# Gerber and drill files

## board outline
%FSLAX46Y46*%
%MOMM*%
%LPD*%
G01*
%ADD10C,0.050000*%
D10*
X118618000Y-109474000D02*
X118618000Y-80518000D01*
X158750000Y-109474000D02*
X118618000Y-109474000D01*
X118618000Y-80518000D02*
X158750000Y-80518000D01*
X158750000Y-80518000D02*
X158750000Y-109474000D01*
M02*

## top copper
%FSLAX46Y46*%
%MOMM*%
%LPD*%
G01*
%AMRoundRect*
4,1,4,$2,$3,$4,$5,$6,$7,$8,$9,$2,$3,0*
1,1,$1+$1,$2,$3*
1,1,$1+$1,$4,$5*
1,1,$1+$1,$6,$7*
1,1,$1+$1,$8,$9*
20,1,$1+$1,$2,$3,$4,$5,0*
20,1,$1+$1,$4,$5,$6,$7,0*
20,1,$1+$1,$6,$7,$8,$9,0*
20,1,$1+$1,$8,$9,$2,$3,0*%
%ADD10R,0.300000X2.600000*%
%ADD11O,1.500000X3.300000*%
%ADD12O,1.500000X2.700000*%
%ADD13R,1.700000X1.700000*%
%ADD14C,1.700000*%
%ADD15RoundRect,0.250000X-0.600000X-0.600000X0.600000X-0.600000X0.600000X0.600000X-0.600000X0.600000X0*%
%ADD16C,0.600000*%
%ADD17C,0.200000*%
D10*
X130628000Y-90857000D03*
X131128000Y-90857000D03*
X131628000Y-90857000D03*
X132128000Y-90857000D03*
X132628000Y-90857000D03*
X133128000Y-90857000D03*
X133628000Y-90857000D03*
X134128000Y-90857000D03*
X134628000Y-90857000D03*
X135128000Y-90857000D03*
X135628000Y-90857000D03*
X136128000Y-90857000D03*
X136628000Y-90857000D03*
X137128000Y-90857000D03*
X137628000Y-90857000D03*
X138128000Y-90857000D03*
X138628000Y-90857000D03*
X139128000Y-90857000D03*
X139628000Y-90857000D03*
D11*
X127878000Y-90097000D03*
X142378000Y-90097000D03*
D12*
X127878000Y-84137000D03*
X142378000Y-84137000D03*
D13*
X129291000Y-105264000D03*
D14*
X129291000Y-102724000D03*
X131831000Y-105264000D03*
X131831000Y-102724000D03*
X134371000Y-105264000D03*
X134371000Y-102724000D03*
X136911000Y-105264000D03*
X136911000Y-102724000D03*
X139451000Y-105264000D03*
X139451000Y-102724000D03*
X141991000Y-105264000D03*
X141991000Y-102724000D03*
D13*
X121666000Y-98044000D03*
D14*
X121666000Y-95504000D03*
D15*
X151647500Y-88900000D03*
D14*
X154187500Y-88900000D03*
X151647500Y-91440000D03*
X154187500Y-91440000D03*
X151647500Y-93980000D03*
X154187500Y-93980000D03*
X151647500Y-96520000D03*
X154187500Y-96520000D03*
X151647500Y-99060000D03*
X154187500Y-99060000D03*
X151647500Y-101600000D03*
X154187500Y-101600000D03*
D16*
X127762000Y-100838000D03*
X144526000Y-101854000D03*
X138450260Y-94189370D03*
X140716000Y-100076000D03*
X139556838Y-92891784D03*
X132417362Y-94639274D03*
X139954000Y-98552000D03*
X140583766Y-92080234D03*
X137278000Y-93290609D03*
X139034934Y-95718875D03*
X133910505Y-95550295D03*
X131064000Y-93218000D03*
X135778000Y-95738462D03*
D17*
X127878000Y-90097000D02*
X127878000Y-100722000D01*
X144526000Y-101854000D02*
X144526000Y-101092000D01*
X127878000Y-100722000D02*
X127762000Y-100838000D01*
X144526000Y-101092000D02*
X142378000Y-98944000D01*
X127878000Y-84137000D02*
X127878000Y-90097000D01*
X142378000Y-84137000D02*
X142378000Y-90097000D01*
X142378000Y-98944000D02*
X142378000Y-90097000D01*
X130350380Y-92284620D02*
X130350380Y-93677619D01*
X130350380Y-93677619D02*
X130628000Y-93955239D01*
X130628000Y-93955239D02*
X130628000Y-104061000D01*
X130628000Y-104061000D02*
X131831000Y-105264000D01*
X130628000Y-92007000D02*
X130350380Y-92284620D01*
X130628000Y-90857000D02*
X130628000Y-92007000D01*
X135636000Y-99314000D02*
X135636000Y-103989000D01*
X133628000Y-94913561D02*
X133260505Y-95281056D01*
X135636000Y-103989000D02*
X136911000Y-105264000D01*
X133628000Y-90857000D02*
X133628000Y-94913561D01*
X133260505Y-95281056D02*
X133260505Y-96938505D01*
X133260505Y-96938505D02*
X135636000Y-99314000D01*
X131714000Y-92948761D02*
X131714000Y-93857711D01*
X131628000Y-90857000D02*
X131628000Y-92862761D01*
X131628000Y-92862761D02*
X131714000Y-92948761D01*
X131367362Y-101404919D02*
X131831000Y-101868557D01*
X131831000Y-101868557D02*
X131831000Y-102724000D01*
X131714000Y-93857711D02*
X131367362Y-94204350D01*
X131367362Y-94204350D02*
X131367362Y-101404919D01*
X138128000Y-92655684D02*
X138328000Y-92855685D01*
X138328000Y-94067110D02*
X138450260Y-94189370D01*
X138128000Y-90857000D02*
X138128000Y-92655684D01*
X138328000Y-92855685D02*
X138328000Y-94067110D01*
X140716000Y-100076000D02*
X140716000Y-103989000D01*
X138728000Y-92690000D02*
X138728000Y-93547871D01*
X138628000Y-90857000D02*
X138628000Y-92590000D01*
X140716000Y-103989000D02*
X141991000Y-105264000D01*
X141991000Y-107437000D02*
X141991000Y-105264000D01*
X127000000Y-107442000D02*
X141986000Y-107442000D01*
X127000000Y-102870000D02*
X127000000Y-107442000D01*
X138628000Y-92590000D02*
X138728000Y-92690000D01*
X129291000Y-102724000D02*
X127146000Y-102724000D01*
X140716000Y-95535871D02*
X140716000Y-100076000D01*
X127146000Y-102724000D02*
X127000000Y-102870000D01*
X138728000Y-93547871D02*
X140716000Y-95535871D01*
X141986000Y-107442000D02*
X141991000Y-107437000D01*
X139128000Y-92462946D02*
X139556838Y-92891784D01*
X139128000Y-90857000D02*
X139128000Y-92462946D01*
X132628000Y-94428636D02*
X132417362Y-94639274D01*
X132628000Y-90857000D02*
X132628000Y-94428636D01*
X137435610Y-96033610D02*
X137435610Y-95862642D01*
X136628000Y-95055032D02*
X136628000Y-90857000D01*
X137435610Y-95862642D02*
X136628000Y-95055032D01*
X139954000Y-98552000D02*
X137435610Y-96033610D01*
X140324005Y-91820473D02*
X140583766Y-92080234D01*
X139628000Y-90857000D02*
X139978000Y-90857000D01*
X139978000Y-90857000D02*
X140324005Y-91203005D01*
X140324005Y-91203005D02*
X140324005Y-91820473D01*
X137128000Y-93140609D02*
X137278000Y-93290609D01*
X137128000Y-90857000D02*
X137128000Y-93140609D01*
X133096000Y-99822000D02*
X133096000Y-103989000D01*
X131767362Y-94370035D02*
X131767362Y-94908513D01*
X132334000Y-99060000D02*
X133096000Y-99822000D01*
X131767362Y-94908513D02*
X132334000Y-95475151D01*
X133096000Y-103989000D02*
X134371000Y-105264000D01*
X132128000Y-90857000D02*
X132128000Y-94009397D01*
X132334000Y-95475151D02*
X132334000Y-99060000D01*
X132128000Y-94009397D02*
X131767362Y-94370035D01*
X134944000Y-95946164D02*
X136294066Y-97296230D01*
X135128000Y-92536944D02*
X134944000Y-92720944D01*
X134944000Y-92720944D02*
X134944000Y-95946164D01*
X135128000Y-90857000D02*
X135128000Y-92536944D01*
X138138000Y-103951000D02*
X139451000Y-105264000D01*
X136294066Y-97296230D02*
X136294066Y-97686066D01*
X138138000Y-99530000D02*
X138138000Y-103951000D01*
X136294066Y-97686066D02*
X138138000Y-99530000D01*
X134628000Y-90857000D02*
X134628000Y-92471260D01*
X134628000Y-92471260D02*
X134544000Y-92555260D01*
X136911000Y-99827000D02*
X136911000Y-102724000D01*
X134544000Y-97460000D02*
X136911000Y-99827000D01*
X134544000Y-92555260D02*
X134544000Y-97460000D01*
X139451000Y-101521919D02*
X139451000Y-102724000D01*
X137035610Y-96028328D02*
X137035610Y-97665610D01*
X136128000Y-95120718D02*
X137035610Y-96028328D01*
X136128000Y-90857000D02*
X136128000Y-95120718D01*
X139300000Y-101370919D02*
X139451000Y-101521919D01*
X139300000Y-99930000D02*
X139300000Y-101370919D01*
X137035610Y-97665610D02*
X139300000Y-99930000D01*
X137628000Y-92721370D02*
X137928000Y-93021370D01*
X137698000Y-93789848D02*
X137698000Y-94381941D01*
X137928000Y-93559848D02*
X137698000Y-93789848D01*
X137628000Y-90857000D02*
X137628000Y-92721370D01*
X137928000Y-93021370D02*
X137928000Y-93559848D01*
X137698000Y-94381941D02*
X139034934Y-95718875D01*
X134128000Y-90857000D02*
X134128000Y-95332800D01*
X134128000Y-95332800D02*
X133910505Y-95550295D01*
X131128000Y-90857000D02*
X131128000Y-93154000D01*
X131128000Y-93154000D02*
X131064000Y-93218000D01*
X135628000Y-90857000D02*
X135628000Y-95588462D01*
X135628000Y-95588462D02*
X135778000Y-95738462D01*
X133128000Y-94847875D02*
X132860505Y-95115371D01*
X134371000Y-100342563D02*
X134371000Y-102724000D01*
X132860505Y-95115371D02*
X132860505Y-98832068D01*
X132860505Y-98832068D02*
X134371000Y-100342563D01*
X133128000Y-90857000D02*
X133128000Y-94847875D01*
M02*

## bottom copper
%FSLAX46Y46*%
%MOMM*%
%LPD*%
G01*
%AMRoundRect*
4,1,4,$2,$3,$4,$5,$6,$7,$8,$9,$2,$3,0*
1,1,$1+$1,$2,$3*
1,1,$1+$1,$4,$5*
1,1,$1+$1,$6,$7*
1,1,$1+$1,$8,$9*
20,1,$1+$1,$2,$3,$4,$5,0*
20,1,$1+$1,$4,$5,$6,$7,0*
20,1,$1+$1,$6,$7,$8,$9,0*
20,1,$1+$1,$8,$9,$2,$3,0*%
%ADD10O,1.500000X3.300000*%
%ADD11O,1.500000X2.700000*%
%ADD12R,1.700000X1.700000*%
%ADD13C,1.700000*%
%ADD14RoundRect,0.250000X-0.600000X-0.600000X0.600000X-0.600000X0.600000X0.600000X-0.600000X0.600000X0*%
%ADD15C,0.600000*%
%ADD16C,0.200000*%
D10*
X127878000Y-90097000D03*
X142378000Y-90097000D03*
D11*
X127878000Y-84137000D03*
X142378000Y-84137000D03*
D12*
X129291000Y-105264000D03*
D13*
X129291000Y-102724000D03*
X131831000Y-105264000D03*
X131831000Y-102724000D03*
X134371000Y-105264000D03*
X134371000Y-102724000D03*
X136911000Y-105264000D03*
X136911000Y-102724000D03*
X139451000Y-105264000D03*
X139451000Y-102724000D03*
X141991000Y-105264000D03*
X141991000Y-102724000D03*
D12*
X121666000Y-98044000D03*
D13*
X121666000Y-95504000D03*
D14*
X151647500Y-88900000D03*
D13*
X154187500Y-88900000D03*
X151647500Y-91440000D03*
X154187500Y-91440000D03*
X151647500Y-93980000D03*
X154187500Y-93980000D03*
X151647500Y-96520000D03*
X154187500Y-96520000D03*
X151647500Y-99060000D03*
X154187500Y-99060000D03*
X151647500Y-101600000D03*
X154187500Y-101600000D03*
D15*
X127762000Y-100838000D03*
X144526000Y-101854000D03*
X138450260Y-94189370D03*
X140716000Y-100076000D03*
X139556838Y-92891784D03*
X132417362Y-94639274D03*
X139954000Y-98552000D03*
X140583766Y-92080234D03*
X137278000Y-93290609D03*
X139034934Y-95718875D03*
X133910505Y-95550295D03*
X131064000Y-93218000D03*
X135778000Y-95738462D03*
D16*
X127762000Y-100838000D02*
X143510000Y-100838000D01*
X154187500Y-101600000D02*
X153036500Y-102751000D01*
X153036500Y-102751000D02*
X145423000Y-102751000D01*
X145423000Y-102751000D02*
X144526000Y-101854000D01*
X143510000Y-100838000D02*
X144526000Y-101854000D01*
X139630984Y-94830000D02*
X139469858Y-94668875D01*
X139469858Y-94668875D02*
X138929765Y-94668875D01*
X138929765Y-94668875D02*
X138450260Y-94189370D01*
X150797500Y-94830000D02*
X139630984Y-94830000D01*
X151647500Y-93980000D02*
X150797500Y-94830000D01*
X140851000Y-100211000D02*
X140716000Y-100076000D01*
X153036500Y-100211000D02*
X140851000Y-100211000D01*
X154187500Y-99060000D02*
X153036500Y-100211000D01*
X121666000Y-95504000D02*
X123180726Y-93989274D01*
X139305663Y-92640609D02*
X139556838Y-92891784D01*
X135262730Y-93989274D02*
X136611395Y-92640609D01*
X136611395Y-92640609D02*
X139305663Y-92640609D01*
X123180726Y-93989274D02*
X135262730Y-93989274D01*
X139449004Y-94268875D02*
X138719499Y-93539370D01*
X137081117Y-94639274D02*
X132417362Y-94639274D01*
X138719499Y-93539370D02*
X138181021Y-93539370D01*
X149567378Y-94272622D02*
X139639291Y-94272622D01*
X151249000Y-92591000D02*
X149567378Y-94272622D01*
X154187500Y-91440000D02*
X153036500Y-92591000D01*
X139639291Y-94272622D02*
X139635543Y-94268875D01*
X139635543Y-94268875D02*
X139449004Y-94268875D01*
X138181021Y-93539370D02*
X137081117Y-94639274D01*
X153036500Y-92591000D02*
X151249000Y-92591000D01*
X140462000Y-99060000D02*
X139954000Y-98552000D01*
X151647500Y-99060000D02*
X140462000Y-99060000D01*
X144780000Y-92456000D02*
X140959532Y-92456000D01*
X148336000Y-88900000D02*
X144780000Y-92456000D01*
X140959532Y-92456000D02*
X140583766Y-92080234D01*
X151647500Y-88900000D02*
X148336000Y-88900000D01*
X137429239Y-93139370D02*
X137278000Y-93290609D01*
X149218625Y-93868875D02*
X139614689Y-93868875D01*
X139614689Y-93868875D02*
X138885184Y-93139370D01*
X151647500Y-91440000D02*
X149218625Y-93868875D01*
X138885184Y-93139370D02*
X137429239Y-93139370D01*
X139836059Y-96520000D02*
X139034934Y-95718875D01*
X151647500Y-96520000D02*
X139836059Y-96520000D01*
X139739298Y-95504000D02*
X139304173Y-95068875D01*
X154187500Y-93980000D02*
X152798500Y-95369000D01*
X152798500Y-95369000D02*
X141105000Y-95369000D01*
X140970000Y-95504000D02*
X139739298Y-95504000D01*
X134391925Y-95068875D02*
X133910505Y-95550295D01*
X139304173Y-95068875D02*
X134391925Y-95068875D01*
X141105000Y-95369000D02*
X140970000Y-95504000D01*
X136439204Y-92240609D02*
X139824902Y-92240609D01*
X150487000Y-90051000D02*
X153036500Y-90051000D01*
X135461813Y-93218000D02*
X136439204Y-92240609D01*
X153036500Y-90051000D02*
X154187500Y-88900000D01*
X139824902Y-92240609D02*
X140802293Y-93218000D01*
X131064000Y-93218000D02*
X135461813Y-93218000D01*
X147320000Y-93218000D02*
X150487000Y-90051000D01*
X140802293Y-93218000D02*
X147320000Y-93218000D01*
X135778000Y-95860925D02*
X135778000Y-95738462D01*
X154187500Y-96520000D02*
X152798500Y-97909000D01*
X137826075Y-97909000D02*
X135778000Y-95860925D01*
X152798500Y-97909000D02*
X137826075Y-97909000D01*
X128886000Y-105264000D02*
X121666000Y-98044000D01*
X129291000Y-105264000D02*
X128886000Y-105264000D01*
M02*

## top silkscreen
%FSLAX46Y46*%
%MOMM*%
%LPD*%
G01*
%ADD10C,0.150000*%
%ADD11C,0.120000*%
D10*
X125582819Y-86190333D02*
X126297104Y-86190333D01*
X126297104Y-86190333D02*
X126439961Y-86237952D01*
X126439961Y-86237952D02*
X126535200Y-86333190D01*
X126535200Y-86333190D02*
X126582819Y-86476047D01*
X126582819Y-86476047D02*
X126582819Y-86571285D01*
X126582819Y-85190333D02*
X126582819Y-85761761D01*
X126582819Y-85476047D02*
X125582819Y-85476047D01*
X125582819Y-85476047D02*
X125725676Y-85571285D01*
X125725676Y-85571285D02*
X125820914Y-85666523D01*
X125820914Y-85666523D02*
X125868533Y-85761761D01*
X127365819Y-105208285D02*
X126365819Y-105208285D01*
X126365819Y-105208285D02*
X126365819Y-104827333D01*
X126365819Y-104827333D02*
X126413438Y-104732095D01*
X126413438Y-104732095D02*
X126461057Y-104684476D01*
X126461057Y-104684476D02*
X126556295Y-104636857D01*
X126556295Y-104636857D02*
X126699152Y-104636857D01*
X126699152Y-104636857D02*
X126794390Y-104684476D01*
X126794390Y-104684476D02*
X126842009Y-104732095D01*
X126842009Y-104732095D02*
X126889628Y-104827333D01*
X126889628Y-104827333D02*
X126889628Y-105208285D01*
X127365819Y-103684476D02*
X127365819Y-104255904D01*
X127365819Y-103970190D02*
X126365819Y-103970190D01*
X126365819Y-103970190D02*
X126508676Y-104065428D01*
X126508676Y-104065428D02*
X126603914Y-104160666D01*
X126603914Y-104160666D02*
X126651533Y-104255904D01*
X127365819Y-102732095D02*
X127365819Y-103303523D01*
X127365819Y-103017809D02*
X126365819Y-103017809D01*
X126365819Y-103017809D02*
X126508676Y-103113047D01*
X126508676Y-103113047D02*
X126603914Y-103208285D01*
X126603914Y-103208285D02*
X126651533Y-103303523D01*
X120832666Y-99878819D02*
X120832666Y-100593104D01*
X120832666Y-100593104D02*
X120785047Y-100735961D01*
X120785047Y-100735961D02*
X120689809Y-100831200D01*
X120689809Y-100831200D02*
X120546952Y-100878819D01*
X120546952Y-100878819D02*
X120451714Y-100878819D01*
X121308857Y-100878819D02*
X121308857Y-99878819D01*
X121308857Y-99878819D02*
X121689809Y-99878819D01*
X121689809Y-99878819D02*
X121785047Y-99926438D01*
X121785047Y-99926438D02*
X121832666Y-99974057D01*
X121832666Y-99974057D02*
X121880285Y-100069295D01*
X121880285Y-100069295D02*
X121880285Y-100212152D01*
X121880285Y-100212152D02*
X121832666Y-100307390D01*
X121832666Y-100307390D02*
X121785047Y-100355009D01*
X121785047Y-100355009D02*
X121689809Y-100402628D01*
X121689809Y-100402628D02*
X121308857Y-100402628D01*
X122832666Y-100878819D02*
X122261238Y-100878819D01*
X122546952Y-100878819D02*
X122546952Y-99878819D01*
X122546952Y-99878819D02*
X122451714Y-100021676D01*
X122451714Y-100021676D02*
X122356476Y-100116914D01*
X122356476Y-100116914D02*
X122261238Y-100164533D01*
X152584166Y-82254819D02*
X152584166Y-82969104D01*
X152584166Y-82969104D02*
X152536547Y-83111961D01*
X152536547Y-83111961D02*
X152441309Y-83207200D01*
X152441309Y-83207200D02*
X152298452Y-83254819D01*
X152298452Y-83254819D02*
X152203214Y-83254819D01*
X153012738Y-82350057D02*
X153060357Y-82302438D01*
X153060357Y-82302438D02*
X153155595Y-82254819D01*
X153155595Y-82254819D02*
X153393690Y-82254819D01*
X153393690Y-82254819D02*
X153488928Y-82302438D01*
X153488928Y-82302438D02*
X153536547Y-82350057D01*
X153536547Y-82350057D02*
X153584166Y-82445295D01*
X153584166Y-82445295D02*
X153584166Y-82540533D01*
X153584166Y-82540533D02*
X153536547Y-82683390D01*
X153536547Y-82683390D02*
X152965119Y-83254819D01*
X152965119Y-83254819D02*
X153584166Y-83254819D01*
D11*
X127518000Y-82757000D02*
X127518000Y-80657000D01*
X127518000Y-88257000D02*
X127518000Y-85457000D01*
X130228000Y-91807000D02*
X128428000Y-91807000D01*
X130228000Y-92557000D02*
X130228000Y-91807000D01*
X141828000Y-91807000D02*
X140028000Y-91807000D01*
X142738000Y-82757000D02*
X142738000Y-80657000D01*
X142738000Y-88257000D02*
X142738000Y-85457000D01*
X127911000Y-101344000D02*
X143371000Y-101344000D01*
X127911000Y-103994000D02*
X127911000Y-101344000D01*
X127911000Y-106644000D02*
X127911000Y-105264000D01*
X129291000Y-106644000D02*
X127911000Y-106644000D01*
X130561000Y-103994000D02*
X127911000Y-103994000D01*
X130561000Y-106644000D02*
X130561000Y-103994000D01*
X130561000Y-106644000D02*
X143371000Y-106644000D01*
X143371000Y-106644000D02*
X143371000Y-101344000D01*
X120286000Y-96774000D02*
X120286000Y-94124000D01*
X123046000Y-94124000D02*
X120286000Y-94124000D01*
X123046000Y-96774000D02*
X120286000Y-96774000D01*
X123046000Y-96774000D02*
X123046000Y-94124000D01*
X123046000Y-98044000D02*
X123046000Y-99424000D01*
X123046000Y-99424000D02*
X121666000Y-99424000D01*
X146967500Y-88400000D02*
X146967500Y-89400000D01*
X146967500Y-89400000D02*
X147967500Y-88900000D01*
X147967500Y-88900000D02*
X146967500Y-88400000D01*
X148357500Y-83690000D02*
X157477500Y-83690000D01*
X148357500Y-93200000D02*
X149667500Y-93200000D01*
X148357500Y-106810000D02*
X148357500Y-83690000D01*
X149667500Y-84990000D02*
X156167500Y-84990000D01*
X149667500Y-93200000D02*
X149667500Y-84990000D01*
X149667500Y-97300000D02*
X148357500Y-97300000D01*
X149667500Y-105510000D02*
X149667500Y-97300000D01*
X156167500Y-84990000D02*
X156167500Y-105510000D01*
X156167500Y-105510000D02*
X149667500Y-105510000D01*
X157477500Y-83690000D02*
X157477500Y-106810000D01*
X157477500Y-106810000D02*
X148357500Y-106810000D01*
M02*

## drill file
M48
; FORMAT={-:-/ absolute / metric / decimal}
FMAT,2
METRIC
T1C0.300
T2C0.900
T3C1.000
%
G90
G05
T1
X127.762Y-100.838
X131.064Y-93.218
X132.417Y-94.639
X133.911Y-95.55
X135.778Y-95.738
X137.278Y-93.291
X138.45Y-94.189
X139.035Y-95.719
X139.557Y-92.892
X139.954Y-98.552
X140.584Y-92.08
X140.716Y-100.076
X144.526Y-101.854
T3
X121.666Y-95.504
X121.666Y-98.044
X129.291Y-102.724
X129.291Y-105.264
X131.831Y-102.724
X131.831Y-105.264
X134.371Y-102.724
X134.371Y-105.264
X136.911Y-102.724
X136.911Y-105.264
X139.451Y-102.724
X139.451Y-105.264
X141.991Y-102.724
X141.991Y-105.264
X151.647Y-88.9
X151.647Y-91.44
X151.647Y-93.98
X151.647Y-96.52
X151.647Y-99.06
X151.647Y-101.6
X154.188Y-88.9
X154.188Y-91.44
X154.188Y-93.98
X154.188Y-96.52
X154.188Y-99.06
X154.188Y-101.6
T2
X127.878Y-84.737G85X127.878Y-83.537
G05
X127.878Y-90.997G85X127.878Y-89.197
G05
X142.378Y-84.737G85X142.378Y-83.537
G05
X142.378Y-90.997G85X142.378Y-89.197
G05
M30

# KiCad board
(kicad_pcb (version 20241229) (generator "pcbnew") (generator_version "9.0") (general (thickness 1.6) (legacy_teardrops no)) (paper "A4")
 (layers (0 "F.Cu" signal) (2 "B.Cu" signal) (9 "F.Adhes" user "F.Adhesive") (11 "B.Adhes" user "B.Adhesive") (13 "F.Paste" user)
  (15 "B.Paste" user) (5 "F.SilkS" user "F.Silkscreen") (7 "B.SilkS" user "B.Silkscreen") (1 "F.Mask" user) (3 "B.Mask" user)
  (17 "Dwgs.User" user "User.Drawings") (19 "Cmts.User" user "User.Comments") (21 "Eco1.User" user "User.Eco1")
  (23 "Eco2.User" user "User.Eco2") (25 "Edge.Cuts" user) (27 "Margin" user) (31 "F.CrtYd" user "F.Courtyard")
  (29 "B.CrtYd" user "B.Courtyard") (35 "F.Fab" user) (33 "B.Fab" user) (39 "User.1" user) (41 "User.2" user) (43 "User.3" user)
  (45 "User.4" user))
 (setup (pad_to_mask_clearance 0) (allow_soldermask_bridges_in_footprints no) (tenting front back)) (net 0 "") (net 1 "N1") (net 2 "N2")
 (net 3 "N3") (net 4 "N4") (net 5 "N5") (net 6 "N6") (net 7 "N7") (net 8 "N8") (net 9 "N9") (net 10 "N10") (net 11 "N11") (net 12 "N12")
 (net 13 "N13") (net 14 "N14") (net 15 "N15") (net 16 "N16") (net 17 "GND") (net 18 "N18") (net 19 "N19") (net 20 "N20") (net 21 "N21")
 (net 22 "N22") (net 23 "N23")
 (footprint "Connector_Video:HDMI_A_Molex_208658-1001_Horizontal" (layer "F.Cu") (at 135.128 87.572 90)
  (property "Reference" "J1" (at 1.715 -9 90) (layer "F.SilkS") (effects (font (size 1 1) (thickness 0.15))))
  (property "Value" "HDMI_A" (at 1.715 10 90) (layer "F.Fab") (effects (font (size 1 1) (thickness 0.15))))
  (fp_line (start 4.815 -7.61) (end 6.915 -7.61) (stroke (width 0.12) (type solid)) (layer "F.SilkS"))
  (fp_line (start -0.685 -7.61) (end 2.115 -7.61) (stroke (width 0.12) (type solid)) (layer "F.SilkS"))
  (fp_line (start -4.235 -4.9) (end -4.235 -6.7) (stroke (width 0.12) (type solid)) (layer "F.SilkS"))
  (fp_line (start -4.985 -4.9) (end -4.235 -4.9) (stroke (width 0.12) (type solid)) (layer "F.SilkS"))
  (fp_line (start -4.235 6.7) (end -4.235 4.9) (stroke (width 0.12) (type solid)) (layer "F.SilkS"))
  (fp_line (start 4.815 7.61) (end 6.915 7.61) (stroke (width 0.12) (type solid)) (layer "F.SilkS"))
  (fp_line (start -0.685 7.61) (end 2.115 7.61) (stroke (width 0.12) (type solid)) (layer "F.SilkS"))
  (pad "1" smd rect (at -3.285 -4.5 90) (size 2.6 0.3) (layers "F.Cu" "F.Mask" "F.Paste") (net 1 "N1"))
  (pad "2" smd rect (at -3.285 -4 90) (size 2.6 0.3) (layers "F.Cu" "F.Mask" "F.Paste") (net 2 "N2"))
  (pad "3" smd rect (at -3.285 -3.5 90) (size 2.6 0.3) (layers "F.Cu" "F.Mask" "F.Paste") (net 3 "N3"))
  (pad "4" smd rect (at -3.285 -3 90) (size 2.6 0.3) (layers "F.Cu" "F.Mask" "F.Paste") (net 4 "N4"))
  (pad "5" smd rect (at -3.285 -2.5 90) (size 2.6 0.3) (layers "F.Cu" "F.Mask" "F.Paste") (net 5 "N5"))
  (pad "6" smd rect (at -3.285 -2 90) (size 2.6 0.3) (layers "F.Cu" "F.Mask" "F.Paste") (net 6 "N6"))
  (pad "7" smd rect (at -3.285 -1.5 90) (size 2.6 0.3) (layers "F.Cu" "F.Mask" "F.Paste") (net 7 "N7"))
  (pad "8" smd rect (at -3.285 -1 90) (size 2.6 0.3) (layers "F.Cu" "F.Mask" "F.Paste") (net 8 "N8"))
  (pad "9" smd rect (at -3.285 -0.5 90) (size 2.6 0.3) (layers "F.Cu" "F.Mask" "F.Paste") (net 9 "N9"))
  (pad "10" smd rect (at -3.285 0 90) (size 2.6 0.3) (layers "F.Cu" "F.Mask" "F.Paste") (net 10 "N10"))
  (pad "11" smd rect (at -3.285 0.5 90) (size 2.6 0.3) (layers "F.Cu" "F.Mask" "F.Paste") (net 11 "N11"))
  (pad "12" smd rect (at -3.285 1 90) (size 2.6 0.3) (layers "F.Cu" "F.Mask" "F.Paste") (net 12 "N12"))
  (pad "13" smd rect (at -3.285 1.5 90) (size 2.6 0.3) (layers "F.Cu" "F.Mask" "F.Paste") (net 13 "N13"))
  (pad "14" smd rect (at -3.285 2 90) (size 2.6 0.3) (layers "F.Cu" "F.Mask" "F.Paste") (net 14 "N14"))
  (pad "15" smd rect (at -3.285 2.5 90) (size 2.6 0.3) (layers "F.Cu" "F.Mask" "F.Paste") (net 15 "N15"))
  (pad "16" smd rect (at -3.285 3 90) (size 2.6 0.3) (layers "F.Cu" "F.Mask" "F.Paste") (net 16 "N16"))
  (pad "17" smd rect (at -3.285 3.5 90) (size 2.6 0.3) (layers "F.Cu" "F.Mask" "F.Paste") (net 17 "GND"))
  (pad "18" smd rect (at -3.285 4 90) (size 2.6 0.3) (layers "F.Cu" "F.Mask" "F.Paste") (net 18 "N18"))
  (pad "19" smd rect (at -3.285 4.5 90) (size 2.6 0.3) (layers "F.Cu" "F.Mask" "F.Paste") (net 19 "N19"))
  (pad "SH" thru_hole oval (at -2.525 -7.25 90) (size 3.3 1.5) (drill oval 2.7 0.9) (layers "*.Cu" "*.Mask") (remove_unused_layers no)
   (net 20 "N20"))
  (pad "SH" thru_hole oval (at -2.525 7.25 90) (size 3.3 1.5) (drill oval 2.7 0.9) (layers "*.Cu" "*.Mask") (remove_unused_layers no)
   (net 20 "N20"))
  (pad "SH" thru_hole oval (at 3.435 -7.25 90) (size 2.7 1.5) (drill oval 2.1 0.9) (layers "*.Cu" "*.Mask") (remove_unused_layers no)
   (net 20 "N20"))
  (pad "SH" thru_hole oval (at 3.435 7.25 90) (size 2.7 1.5) (drill oval 2.1 0.9) (layers "*.Cu" "*.Mask") (remove_unused_layers no)
   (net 20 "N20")))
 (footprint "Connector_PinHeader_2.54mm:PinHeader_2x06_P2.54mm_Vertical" (layer "F.Cu") (at 129.291 105.264 90)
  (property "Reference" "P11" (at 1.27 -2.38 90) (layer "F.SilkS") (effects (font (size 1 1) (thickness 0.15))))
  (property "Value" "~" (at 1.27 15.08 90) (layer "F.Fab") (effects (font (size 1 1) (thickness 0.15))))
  (fp_line (start 3.92 -1.38) (end 3.92 14.08) (stroke (width 0.12) (type solid)) (layer "F.SilkS"))
  (fp_line (start 1.27 -1.38) (end 3.92 -1.38) (stroke (width 0.12) (type solid)) (layer "F.SilkS"))
  (fp_line (start -1.38 -1.38) (end 0 -1.38) (stroke (width 0.12) (type solid)) (layer "F.SilkS"))
  (fp_line (start -1.38 0) (end -1.38 -1.38) (stroke (width 0.12) (type solid)) (layer "F.SilkS"))
  (fp_line (start 1.27 1.27) (end 1.27 -1.38) (stroke (width 0.12) (type solid)) (layer "F.SilkS"))
  (fp_line (start -1.38 1.27) (end 1.27 1.27) (stroke (width 0.12) (type solid)) (layer "F.SilkS"))
  (fp_line (start -1.38 1.27) (end -1.38 14.08) (stroke (width 0.12) (type solid)) (layer "F.SilkS"))
  (fp_line (start -1.38 14.08) (end 3.92 14.08) (stroke (width 0.12) (type solid)) (layer "F.SilkS"))
  (pad "1" thru_hole rect (at 0 0 90) (size 1.7 1.7) (drill 1) (layers "*.Cu" "*.Mask") (remove_unused_layers no) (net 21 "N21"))
  (pad "2" thru_hole circle (at 2.54 0 90) (size 1.7 1.7) (drill 1) (layers "*.Cu" "*.Mask") (remove_unused_layers no) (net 17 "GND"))
  (pad "3" thru_hole circle (at 0 2.54 90) (size 1.7 1.7) (drill 1) (layers "*.Cu" "*.Mask") (remove_unused_layers no) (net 1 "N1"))
  (pad "4" thru_hole circle (at 2.54 2.54 90) (size 1.7 1.7) (drill 1) (layers "*.Cu" "*.Mask") (remove_unused_layers no) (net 3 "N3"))
  (pad "5" thru_hole circle (at 0 5.08 90) (size 1.7 1.7) (drill 1) (layers "*.Cu" "*.Mask") (remove_unused_layers no) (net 4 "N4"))
  (pad "6" thru_hole circle (at 2.54 5.08 90) (size 1.7 1.7) (drill 1) (layers "*.Cu" "*.Mask") (remove_unused_layers no) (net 6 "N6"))
  (pad "7" thru_hole circle (at 0 7.62 90) (size 1.7 1.7) (drill 1) (layers "*.Cu" "*.Mask") (remove_unused_layers no) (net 7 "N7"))
  (pad "8" thru_hole circle (at 2.54 7.62 90) (size 1.7 1.7) (drill 1) (layers "*.Cu" "*.Mask") (remove_unused_layers no) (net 9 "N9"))
  (pad "9" thru_hole circle (at 0 10.16 90) (size 1.7 1.7) (drill 1) (layers "*.Cu" "*.Mask") (remove_unused_layers no) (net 10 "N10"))
  (pad "10" thru_hole circle (at 2.54 10.16 90) (size 1.7 1.7) (drill 1) (layers "*.Cu" "*.Mask") (remove_unused_layers no) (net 12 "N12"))
  (pad "11" thru_hole circle (at 0 12.7 90) (size 1.7 1.7) (drill 1) (layers "*.Cu" "*.Mask") (remove_unused_layers no) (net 17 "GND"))
  (pad "12" thru_hole circle (at 2.54 12.7 90) (size 1.7 1.7) (drill 1) (layers "*.Cu" "*.Mask") (remove_unused_layers no) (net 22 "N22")))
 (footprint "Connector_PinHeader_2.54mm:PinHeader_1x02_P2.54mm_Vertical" (layer "F.Cu") (at 121.666 98.044 180)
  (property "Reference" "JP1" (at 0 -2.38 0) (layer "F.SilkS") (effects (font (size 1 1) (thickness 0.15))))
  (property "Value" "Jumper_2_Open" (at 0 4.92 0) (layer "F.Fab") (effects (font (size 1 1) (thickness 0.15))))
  (fp_line (start 1.38 1.27) (end 1.38 3.92) (stroke (width 0.12) (type solid)) (layer "F.SilkS"))
  (fp_line (start -1.38 3.92) (end 1.38 3.92) (stroke (width 0.12) (type solid)) (layer "F.SilkS"))
  (fp_line (start -1.38 1.27) (end 1.38 1.27) (stroke (width 0.12) (type solid)) (layer "F.SilkS"))
  (fp_line (start -1.38 1.27) (end -1.38 3.92) (stroke (width 0.12) (type solid)) (layer "F.SilkS"))
  (fp_line (start -1.38 0) (end -1.38 -1.38) (stroke (width 0.12) (type solid)) (layer "F.SilkS"))
  (fp_line (start -1.38 -1.38) (end 0 -1.38) (stroke (width 0.12) (type solid)) (layer "F.SilkS"))
  (pad "1" thru_hole rect (at 0 0 180) (size 1.7 1.7) (drill 1) (layers "*.Cu" "*.Mask") (remove_unused_layers no) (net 21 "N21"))
  (pad "2" thru_hole circle (at 0 2.54 180) (size 1.7 1.7) (drill 1) (layers "*.Cu" "*.Mask") (remove_unused_layers no) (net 18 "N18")))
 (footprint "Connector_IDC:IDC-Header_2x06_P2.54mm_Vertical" (layer "F.Cu") (at 151.6475 88.9)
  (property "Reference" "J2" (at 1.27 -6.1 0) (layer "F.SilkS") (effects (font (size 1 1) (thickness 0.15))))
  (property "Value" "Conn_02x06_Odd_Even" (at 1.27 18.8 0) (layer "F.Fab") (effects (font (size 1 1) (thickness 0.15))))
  (fp_line (start -4.68 -0.5) (end -4.68 0.5) (stroke (width 0.12) (type solid)) (layer "F.SilkS"))
  (fp_line (start -4.68 0.5) (end -3.68 0) (stroke (width 0.12) (type solid)) (layer "F.SilkS"))
  (fp_line (start -3.68 0) (end -4.68 -0.5) (stroke (width 0.12) (type solid)) (layer "F.SilkS"))
  (fp_line (start -3.29 -5.21) (end 5.83 -5.21) (stroke (width 0.12) (type solid)) (layer "F.SilkS"))
  (fp_line (start -3.29 4.3) (end -1.98 4.3) (stroke (width 0.12) (type solid)) (layer "F.SilkS"))
  (fp_line (start -3.29 17.91) (end -3.29 -5.21) (stroke (width 0.12) (type solid)) (layer "F.SilkS"))
  (fp_line (start -1.98 -3.91) (end 4.52 -3.91) (stroke (width 0.12) (type solid)) (layer "F.SilkS"))
  (fp_line (start -1.98 4.3) (end -1.98 -3.91) (stroke (width 0.12) (type solid)) (layer "F.SilkS"))
  (fp_line (start -1.98 8.4) (end -3.29 8.4) (stroke (width 0.12) (type solid)) (layer "F.SilkS"))
  (fp_line (start -1.98 16.61) (end -1.98 8.4) (stroke (width 0.12) (type solid)) (layer "F.SilkS"))
  (fp_line (start 4.52 -3.91) (end 4.52 16.61) (stroke (width 0.12) (type solid)) (layer "F.SilkS"))
  (fp_line (start 4.52 16.61) (end -1.98 16.61) (stroke (width 0.12) (type solid)) (layer "F.SilkS"))
  (fp_line (start 5.83 -5.21) (end 5.83 17.91) (stroke (width 0.12) (type solid)) (layer "F.SilkS"))
  (fp_line (start 5.83 17.91) (end -3.29 17.91) (stroke (width 0.12) (type solid)) (layer "F.SilkS"))
  (pad "1" thru_hole roundrect (at 0 0) (size 1.7 1.7) (drill 1) (layers "*.Cu" "*.Mask") (remove_unused_layers no)
   (roundrect_rratio 0.147059) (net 19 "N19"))
  (pad "2" thru_hole circle (at 2.54 0) (size 1.7 1.7) (drill 1) (layers "*.Cu" "*.Mask") (remove_unused_layers no) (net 2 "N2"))
  (pad "3" thru_hole circle (at 0 2.54) (size 1.7 1.7) (drill 1) (layers "*.Cu" "*.Mask") (remove_unused_layers no) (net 14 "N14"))
  (pad "4" thru_hole circle (at 2.54 2.54) (size 1.7 1.7) (drill 1) (layers "*.Cu" "*.Mask") (remove_unused_layers no) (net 5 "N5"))
  (pad "5" thru_hole circle (at 0 5.08) (size 1.7 1.7) (drill 1) (layers "*.Cu" "*.Mask") (remove_unused_layers no) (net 16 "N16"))
  (pad "6" thru_hole circle (at 2.54 5.08) (size 1.7 1.7) (drill 1) (layers "*.Cu" "*.Mask") (remove_unused_layers no) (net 8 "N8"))
  (pad "7" thru_hole circle (at 0 7.62) (size 1.7 1.7) (drill 1) (layers "*.Cu" "*.Mask") (remove_unused_layers no) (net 15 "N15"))
  (pad "8" thru_hole circle (at 2.54 7.62) (size 1.7 1.7) (drill 1) (layers "*.Cu" "*.Mask") (remove_unused_layers no) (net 11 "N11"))
  (pad "9" thru_hole circle (at 0 10.16) (size 1.7 1.7) (drill 1) (layers "*.Cu" "*.Mask") (remove_unused_layers no) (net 13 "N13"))
  (pad "10" thru_hole circle (at 2.54 10.16) (size 1.7 1.7) (drill 1) (layers "*.Cu" "*.Mask") (remove_unused_layers no) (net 17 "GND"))
  (pad "11" thru_hole circle (at 0 12.7) (size 1.7 1.7) (drill 1) (layers "*.Cu" "*.Mask") (remove_unused_layers no) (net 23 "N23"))
  (pad "12" thru_hole circle (at 2.54 12.7) (size 1.7 1.7) (drill 1) (layers "*.Cu" "*.Mask") (remove_unused_layers no) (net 20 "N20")))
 (gr_line (start 118.618 109.474) (end 118.618 80.518) (stroke (width 0.05) (type default)) (layer "Edge.Cuts"))
 (gr_line (start 158.75 109.474) (end 118.618 109.474) (stroke (width 0.05) (type default)) (layer "Edge.Cuts"))
 (gr_line (start 118.618 80.518) (end 158.75 80.518) (stroke (width 0.05) (type default)) (layer "Edge.Cuts"))
 (gr_line (start 158.75 80.518) (end 158.75 109.474) (stroke (width 0.05) (type default)) (layer "Edge.Cuts"))
 (segment (start 127.878 90.097) (end 127.878 100.722) (width 0.2) (layer "F.Cu") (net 20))
 (segment (start 144.526 101.854) (end 144.526 101.092) (width 0.2) (layer "F.Cu") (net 20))
 (segment (start 127.878 100.722) (end 127.762 100.838) (width 0.2) (layer "F.Cu") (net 20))
 (segment (start 144.526 101.092) (end 142.378 98.944) (width 0.2) (layer "F.Cu") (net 20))
 (segment (start 127.878 84.137) (end 127.878 90.097) (width 0.2) (layer "F.Cu") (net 20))
 (segment (start 142.378 84.137) (end 142.378 90.097) (width 0.2) (layer "F.Cu") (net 20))
 (segment (start 142.378 98.944) (end 142.378 90.097) (width 0.2) (layer "F.Cu") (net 20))
 (via (at 127.762 100.838) (size 0.6) (drill 0.3) (layers "F.Cu" "B.Cu") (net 20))
 (via (at 144.526 101.854) (size 0.6) (drill 0.3) (layers "F.Cu" "B.Cu") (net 20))
 (segment (start 127.762 100.838) (end 143.51 100.838) (width 0.2) (layer "B.Cu") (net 20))
 (segment (start 154.1875 101.6) (end 153.0365 102.751) (width 0.2) (layer "B.Cu") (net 20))
 (segment (start 153.0365 102.751) (end 145.423 102.751) (width 0.2) (layer "B.Cu") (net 20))
 (segment (start 145.423 102.751) (end 144.526 101.854) (width 0.2) (layer "B.Cu") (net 20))
 (segment (start 143.51 100.838) (end 144.526 101.854) (width 0.2) (layer "B.Cu") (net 20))
 (segment (start 130.35038 92.28462) (end 130.35038 93.677619) (width 0.2) (layer "F.Cu") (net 1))
 (segment (start 130.35038 93.677619) (end 130.628 93.955239) (width 0.2) (layer "F.Cu") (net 1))
 (segment (start 130.628 93.955239) (end 130.628 104.061) (width 0.2) (layer "F.Cu") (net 1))
 (segment (start 130.628 104.061) (end 131.831 105.264) (width 0.2) (layer "F.Cu") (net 1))
 (segment (start 130.628 92.007) (end 130.35038 92.28462) (width 0.2) (layer "F.Cu") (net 1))
 (segment (start 130.628 90.857) (end 130.628 92.007) (width 0.2) (layer "F.Cu") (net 1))
 (segment (start 135.636 99.314) (end 135.636 103.989) (width 0.2) (layer "F.Cu") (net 7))
 (segment (start 133.628 94.913561) (end 133.260505 95.281056) (width 0.2) (layer "F.Cu") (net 7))
 (segment (start 135.636 103.989) (end 136.911 105.264) (width 0.2) (layer "F.Cu") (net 7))
 (segment (start 133.628 90.857) (end 133.628 94.913561) (width 0.2) (layer "F.Cu") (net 7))
 (segment (start 133.260505 95.281056) (end 133.260505 96.938505) (width 0.2) (layer "F.Cu") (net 7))
 (segment (start 133.260505 96.938505) (end 135.636 99.314) (width 0.2) (layer "F.Cu") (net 7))
 (segment (start 131.714 92.948761) (end 131.714 93.857711) (width 0.2) (layer "F.Cu") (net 3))
 (segment (start 131.628 90.857) (end 131.628 92.862761) (width 0.2) (layer "F.Cu") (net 3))
 (segment (start 131.628 92.862761) (end 131.714 92.948761) (width 0.2) (layer "F.Cu") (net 3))
 (segment (start 131.367362 101.404919) (end 131.831 101.868557) (width 0.2) (layer "F.Cu") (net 3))
 (segment (start 131.831 101.868557) (end 131.831 102.724) (width 0.2) (layer "F.Cu") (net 3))
 (segment (start 131.714 93.857711) (end 131.367362 94.20435) (width 0.2) (layer "F.Cu") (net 3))
 (segment (start 131.367362 94.20435) (end 131.367362 101.404919) (width 0.2) (layer "F.Cu") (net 3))
 (segment (start 138.128 92.655684) (end 138.328 92.855685) (width 0.2) (layer "F.Cu") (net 16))
 (segment (start 138.328 94.06711) (end 138.45026 94.18937) (width 0.2) (layer "F.Cu") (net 16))
 (segment (start 138.128 90.857) (end 138.128 92.655684) (width 0.2) (layer "F.Cu") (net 16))
 (segment (start 138.328 92.855685) (end 138.328 94.06711) (width 0.2) (layer "F.Cu") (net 16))
 (via (at 138.45026 94.18937) (size 0.6) (drill 0.3) (layers "F.Cu" "B.Cu") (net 16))
 (segment (start 139.630984 94.83) (end 139.469858 94.668875) (width 0.2) (layer "B.Cu") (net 16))
 (segment (start 139.469858 94.668875) (end 138.929765 94.668875) (width 0.2) (layer "B.Cu") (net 16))
 (segment (start 138.929765 94.668875) (end 138.45026 94.18937) (width 0.2) (layer "B.Cu") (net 16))
 (segment (start 150.7975 94.83) (end 139.630984 94.83) (width 0.2) (layer "B.Cu") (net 16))
 (segment (start 151.6475 93.98) (end 150.7975 94.83) (width 0.2) (layer "B.Cu") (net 16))
 (segment (start 140.716 100.076) (end 140.716 103.989) (width 0.2) (layer "F.Cu") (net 17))
 (segment (start 138.728 92.69) (end 138.728 93.547871) (width 0.2) (layer "F.Cu") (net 17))
 (segment (start 138.628 90.857) (end 138.628 92.59) (width 0.2) (layer "F.Cu") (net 17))
 (segment (start 140.716 103.989) (end 141.991 105.264) (width 0.2) (layer "F.Cu") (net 17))
 (segment (start 141.991 107.437) (end 141.991 105.264) (width 0.2) (layer "F.Cu") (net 17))
 (segment (start 127 107.442) (end 141.986 107.442) (width 0.2) (layer "F.Cu") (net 17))
 (segment (start 127 102.87) (end 127 107.442) (width 0.2) (layer "F.Cu") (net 17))
 (segment (start 138.628 92.59) (end 138.728 92.69) (width 0.2) (layer "F.Cu") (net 17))
 (segment (start 129.291 102.724) (end 127.146 102.724) (width 0.2) (layer "F.Cu") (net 17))
 (segment (start 140.716 95.535871) (end 140.716 100.076) (width 0.2) (layer "F.Cu") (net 17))
 (segment (start 127.146 102.724) (end 127 102.87) (width 0.2) (layer "F.Cu") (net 17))
 (segment (start 138.728 93.547871) (end 140.716 95.535871) (width 0.2) (layer "F.Cu") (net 17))
 (segment (start 141.986 107.442) (end 141.991 107.437) (width 0.2) (layer "F.Cu") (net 17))
 (via (at 140.716 100.076) (size 0.6) (drill 0.3) (layers "F.Cu" "B.Cu") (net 17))
 (segment (start 140.851 100.211) (end 140.716 100.076) (width 0.2) (layer "B.Cu") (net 17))
 (segment (start 153.0365 100.211) (end 140.851 100.211) (width 0.2) (layer "B.Cu") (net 17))
 (segment (start 154.1875 99.06) (end 153.0365 100.211) (width 0.2) (layer "B.Cu") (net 17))
 (segment (start 139.128 92.462946) (end 139.556838 92.891784) (width 0.2) (layer "F.Cu") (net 18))
 (segment (start 139.128 90.857) (end 139.128 92.462946) (width 0.2) (layer "F.Cu") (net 18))
 (via (at 139.556838 92.891784) (size 0.6) (drill 0.3) (layers "F.Cu" "B.Cu") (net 18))
 (segment (start 121.666 95.504) (end 123.180726 93.989274) (width 0.2) (layer "B.Cu") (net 18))
 (segment (start 139.305663 92.640609) (end 139.556838 92.891784) (width 0.2) (layer "B.Cu") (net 18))
 (segment (start 135.26273 93.989274) (end 136.611395 92.640609) (width 0.2) (layer "B.Cu") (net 18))
 (segment (start 136.611395 92.640609) (end 139.305663 92.640609) (width 0.2) (layer "B.Cu") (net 18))
 (segment (start 123.180726 93.989274) (end 135.26273 93.989274) (width 0.2) (layer "B.Cu") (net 18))
 (segment (start 132.628 94.428636) (end 132.417362 94.639274) (width 0.2) (layer "F.Cu") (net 5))
 (segment (start 132.628 90.857) (end 132.628 94.428636) (width 0.2) (layer "F.Cu") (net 5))
 (via (at 132.417362 94.639274) (size 0.6) (drill 0.3) (layers "F.Cu" "B.Cu") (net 5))
 (segment (start 139.449004 94.268875) (end 138.719499 93.53937) (width 0.2) (layer "B.Cu") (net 5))
 (segment (start 137.081117 94.639274) (end 132.417362 94.639274) (width 0.2) (layer "B.Cu") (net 5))
 (segment (start 138.719499 93.53937) (end 138.181021 93.53937) (width 0.2) (layer "B.Cu") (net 5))
 (segment (start 149.567378 94.272622) (end 139.639291 94.272622) (width 0.2) (layer "B.Cu") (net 5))
 (segment (start 151.249 92.591) (end 149.567378 94.272622) (width 0.2) (layer "B.Cu") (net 5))
 (segment (start 154.1875 91.44) (end 153.0365 92.591) (width 0.2) (layer "B.Cu") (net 5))
 (segment (start 139.639291 94.272622) (end 139.635543 94.268875) (width 0.2) (layer "B.Cu") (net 5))
 (segment (start 139.635543 94.268875) (end 139.449004 94.268875) (width 0.2) (layer "B.Cu") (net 5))
 (segment (start 138.181021 93.53937) (end 137.081117 94.639274) (width 0.2) (layer "B.Cu") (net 5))
 (segment (start 153.0365 92.591) (end 151.249 92.591) (width 0.2) (layer "B.Cu") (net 5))
 (segment (start 137.43561 96.03361) (end 137.43561 95.862642) (width 0.2) (layer "F.Cu") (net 13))
 (segment (start 136.628 95.055032) (end 136.628 90.857) (width 0.2) (layer "F.Cu") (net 13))
 (segment (start 137.43561 95.862642) (end 136.628 95.055032) (width 0.2) (layer "F.Cu") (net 13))
 (segment (start 139.954 98.552) (end 137.43561 96.03361) (width 0.2) (layer "F.Cu") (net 13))
 (via (at 139.954 98.552) (size 0.6) (drill 0.3) (layers "F.Cu" "B.Cu") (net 13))
 (segment (start 140.462 99.06) (end 139.954 98.552) (width 0.2) (layer "B.Cu") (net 13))
 (segment (start 151.6475 99.06) (end 140.462 99.06) (width 0.2) (layer "B.Cu") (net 13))
 (segment (start 140.324005 91.820473) (end 140.583766 92.080234) (width 0.2) (layer "F.Cu") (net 19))
 (segment (start 139.628 90.857) (end 139.978 90.857) (width 0.2) (layer "F.Cu") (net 19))
 (segment (start 139.978 90.857) (end 140.324005 91.203005) (width 0.2) (layer "F.Cu") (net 19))
 (segment (start 140.324005 91.203005) (end 140.324005 91.820473) (width 0.2) (layer "F.Cu") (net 19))
 (via (at 140.583766 92.080234) (size 0.6) (drill 0.3) (layers "F.Cu" "B.Cu") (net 19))
 (segment (start 144.78 92.456) (end 140.959532 92.456) (width 0.2) (layer "B.Cu") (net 19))
 (segment (start 148.336 88.9) (end 144.78 92.456) (width 0.2) (layer "B.Cu") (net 19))
 (segment (start 140.959532 92.456) (end 140.583766 92.080234) (width 0.2) (layer "B.Cu") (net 19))
 (segment (start 151.6475 88.9) (end 148.336 88.9) (width 0.2) (layer "B.Cu") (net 19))
 (segment (start 137.128 93.140609) (end 137.278 93.290609) (width 0.2) (layer "F.Cu") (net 14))
 (segment (start 137.128 90.857) (end 137.128 93.140609) (width 0.2) (layer "F.Cu") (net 14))
 (via (at 137.278 93.290609) (size 0.6) (drill 0.3) (layers "F.Cu" "B.Cu") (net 14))
 (segment (start 137.429239 93.13937) (end 137.278 93.290609) (width 0.2) (layer "B.Cu") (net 14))
 (segment (start 149.218625 93.868875) (end 139.614689 93.868875) (width 0.2) (layer "B.Cu") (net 14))
 (segment (start 139.614689 93.868875) (end 138.885184 93.13937) (width 0.2) (layer "B.Cu") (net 14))
 (segment (start 151.6475 91.44) (end 149.218625 93.868875) (width 0.2) (layer "B.Cu") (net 14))
 (segment (start 138.885184 93.13937) (end 137.429239 93.13937) (width 0.2) (layer "B.Cu") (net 14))
 (segment (start 133.096 99.822) (end 133.096 103.989) (width 0.2) (layer "F.Cu") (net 4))
 (segment (start 131.767362 94.370035) (end 131.767362 94.908513) (width 0.2) (layer "F.Cu") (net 4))
 (segment (start 132.334 99.06) (end 133.096 99.822) (width 0.2) (layer "F.Cu") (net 4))
 (segment (start 131.767362 94.908513) (end 132.334 95.475151) (width 0.2) (layer "F.Cu") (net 4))
 (segment (start 133.096 103.989) (end 134.371 105.264) (width 0.2) (layer "F.Cu") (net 4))
 (segment (start 132.128 90.857) (end 132.128 94.009397) (width 0.2) (layer "F.Cu") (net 4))
 (segment (start 132.334 95.475151) (end 132.334 99.06) (width 0.2) (layer "F.Cu") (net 4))
 (segment (start 132.128 94.009397) (end 131.767362 94.370035) (width 0.2) (layer "F.Cu") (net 4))
 (segment (start 134.944 95.946164) (end 136.294066 97.29623) (width 0.2) (layer "F.Cu") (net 10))
 (segment (start 135.128 92.536944) (end 134.944 92.720944) (width 0.2) (layer "F.Cu") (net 10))
 (segment (start 134.944 92.720944) (end 134.944 95.946164) (width 0.2) (layer "F.Cu") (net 10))
 (segment (start 135.128 90.857) (end 135.128 92.536944) (width 0.2) (layer "F.Cu") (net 10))
 (segment (start 138.138 103.951) (end 139.451 105.264) (width 0.2) (layer "F.Cu") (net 10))
 (segment (start 136.294066 97.29623) (end 136.294066 97.686066) (width 0.2) (layer "F.Cu") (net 10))
 (segment (start 138.138 99.53) (end 138.138 103.951) (width 0.2) (layer "F.Cu") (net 10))
 (segment (start 136.294066 97.686066) (end 138.138 99.53) (width 0.2) (layer "F.Cu") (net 10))
 (segment (start 134.628 90.857) (end 134.628 92.47126) (width 0.2) (layer "F.Cu") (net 9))
 (segment (start 134.628 92.47126) (end 134.544 92.55526) (width 0.2) (layer "F.Cu") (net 9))
 (segment (start 136.911 99.827) (end 136.911 102.724) (width 0.2) (layer "F.Cu") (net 9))
 (segment (start 134.544 97.46) (end 136.911 99.827) (width 0.2) (layer "F.Cu") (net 9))
 (segment (start 134.544 92.55526) (end 134.544 97.46) (width 0.2) (layer "F.Cu") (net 9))
 (segment (start 139.451 101.521919) (end 139.451 102.724) (width 0.2) (layer "F.Cu") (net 12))
 (segment (start 137.03561 96.028328) (end 137.03561 97.66561) (width 0.2) (layer "F.Cu") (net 12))
 (segment (start 136.128 95.120718) (end 137.03561 96.028328) (width 0.2) (layer "F.Cu") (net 12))
 (segment (start 136.128 90.857) (end 136.128 95.120718) (width 0.2) (layer "F.Cu") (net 12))
 (segment (start 139.3 101.370919) (end 139.451 101.521919) (width 0.2) (layer "F.Cu") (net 12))
 (segment (start 139.3 99.93) (end 139.3 101.370919) (width 0.2) (layer "F.Cu") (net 12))
 (segment (start 137.03561 97.66561) (end 139.3 99.93) (width 0.2) (layer "F.Cu") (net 12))
 (segment (start 137.628 92.72137) (end 137.928 93.02137) (width 0.2) (layer "F.Cu") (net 15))
 (segment (start 137.698 93.789848) (end 137.698 94.381941) (width 0.2) (layer "F.Cu") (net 15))
 (segment (start 137.928 93.559848) (end 137.698 93.789848) (width 0.2) (layer "F.Cu") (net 15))
 (segment (start 137.628 90.857) (end 137.628 92.72137) (width 0.2) (layer "F.Cu") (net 15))
 (segment (start 137.928 93.02137) (end 137.928 93.559848) (width 0.2) (layer "F.Cu") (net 15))
 (segment (start 137.698 94.381941) (end 139.034934 95.718875) (width 0.2) (layer "F.Cu") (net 15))
 (via (at 139.034934 95.718875) (size 0.6) (drill 0.3) (layers "F.Cu" "B.Cu") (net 15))
 (segment (start 139.836059 96.52) (end 139.034934 95.718875) (width 0.2) (layer "B.Cu") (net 15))
 (segment (start 151.6475 96.52) (end 139.836059 96.52) (width 0.2) (layer "B.Cu") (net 15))
 (segment (start 134.128 90.857) (end 134.128 95.3328) (width 0.2) (layer "F.Cu") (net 8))
 (segment (start 134.128 95.3328) (end 133.910505 95.550295) (width 0.2) (layer "F.Cu") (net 8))
 (via (at 133.910505 95.550295) (size 0.6) (drill 0.3) (layers "F.Cu" "B.Cu") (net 8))
 (segment (start 139.739298 95.504) (end 139.304173 95.068875) (width 0.2) (layer "B.Cu") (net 8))
 (segment (start 154.1875 93.98) (end 152.7985 95.369) (width 0.2) (layer "B.Cu") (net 8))
 (segment (start 152.7985 95.369) (end 141.105 95.369) (width 0.2) (layer "B.Cu") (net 8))
 (segment (start 140.97 95.504) (end 139.739298 95.504) (width 0.2) (layer "B.Cu") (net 8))
 (segment (start 134.391925 95.068875) (end 133.910505 95.550295) (width 0.2) (layer "B.Cu") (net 8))
 (segment (start 139.304173 95.068875) (end 134.391925 95.068875) (width 0.2) (layer "B.Cu") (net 8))
 (segment (start 141.105 95.369) (end 140.97 95.504) (width 0.2) (layer "B.Cu") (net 8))
 (segment (start 131.128 90.857) (end 131.128 93.154) (width 0.2) (layer "F.Cu") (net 2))
 (segment (start 131.128 93.154) (end 131.064 93.218) (width 0.2) (layer "F.Cu") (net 2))
 (via (at 131.064 93.218) (size 0.6) (drill 0.3) (layers "F.Cu" "B.Cu") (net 2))
 (segment (start 136.439204 92.240609) (end 139.824902 92.240609) (width 0.2) (layer "B.Cu") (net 2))
 (segment (start 150.487 90.051) (end 153.0365 90.051) (width 0.2) (layer "B.Cu") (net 2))
 (segment (start 135.461813 93.218) (end 136.439204 92.240609) (width 0.2) (layer "B.Cu") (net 2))
 (segment (start 153.0365 90.051) (end 154.1875 88.9) (width 0.2) (layer "B.Cu") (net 2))
 (segment (start 139.824902 92.240609) (end 140.802293 93.218) (width 0.2) (layer "B.Cu") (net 2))
 (segment (start 131.064 93.218) (end 135.461813 93.218) (width 0.2) (layer "B.Cu") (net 2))
 (segment (start 147.32 93.218) (end 150.487 90.051) (width 0.2) (layer "B.Cu") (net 2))
 (segment (start 140.802293 93.218) (end 147.32 93.218) (width 0.2) (layer "B.Cu") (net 2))
 (segment (start 135.628 90.857) (end 135.628 95.588462) (width 0.2) (layer "F.Cu") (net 11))
 (segment (start 135.628 95.588462) (end 135.778 95.738462) (width 0.2) (layer "F.Cu") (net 11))
 (via (at 135.778 95.738462) (size 0.6) (drill 0.3) (layers "F.Cu" "B.Cu") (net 11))
 (segment (start 135.778 95.860925) (end 135.778 95.738462) (width 0.2) (layer "B.Cu") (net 11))
 (segment (start 154.1875 96.52) (end 152.7985 97.909) (width 0.2) (layer "B.Cu") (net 11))
 (segment (start 137.826075 97.909) (end 135.778 95.860925) (width 0.2) (layer "B.Cu") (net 11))
 (segment (start 152.7985 97.909) (end 137.826075 97.909) (width 0.2) (layer "B.Cu") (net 11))
 (segment (start 133.128 94.847875) (end 132.860505 95.115371) (width 0.2) (layer "F.Cu") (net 6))
 (segment (start 134.371 100.342563) (end 134.371 102.724) (width 0.2) (layer "F.Cu") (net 6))
 (segment (start 132.860505 95.115371) (end 132.860505 98.832068) (width 0.2) (layer "F.Cu") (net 6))
 (segment (start 132.860505 98.832068) (end 134.371 100.342563) (width 0.2) (layer "F.Cu") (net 6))
 (segment (start 133.128 90.857) (end 133.128 94.847875) (width 0.2) (layer "F.Cu") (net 6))
 (segment (start 128.886 105.264) (end 121.666 98.044) (width 0.2) (layer "B.Cu") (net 21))
 (segment (start 129.291 105.264) (end 128.886 105.264) (width 0.2) (layer "B.Cu") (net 21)))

